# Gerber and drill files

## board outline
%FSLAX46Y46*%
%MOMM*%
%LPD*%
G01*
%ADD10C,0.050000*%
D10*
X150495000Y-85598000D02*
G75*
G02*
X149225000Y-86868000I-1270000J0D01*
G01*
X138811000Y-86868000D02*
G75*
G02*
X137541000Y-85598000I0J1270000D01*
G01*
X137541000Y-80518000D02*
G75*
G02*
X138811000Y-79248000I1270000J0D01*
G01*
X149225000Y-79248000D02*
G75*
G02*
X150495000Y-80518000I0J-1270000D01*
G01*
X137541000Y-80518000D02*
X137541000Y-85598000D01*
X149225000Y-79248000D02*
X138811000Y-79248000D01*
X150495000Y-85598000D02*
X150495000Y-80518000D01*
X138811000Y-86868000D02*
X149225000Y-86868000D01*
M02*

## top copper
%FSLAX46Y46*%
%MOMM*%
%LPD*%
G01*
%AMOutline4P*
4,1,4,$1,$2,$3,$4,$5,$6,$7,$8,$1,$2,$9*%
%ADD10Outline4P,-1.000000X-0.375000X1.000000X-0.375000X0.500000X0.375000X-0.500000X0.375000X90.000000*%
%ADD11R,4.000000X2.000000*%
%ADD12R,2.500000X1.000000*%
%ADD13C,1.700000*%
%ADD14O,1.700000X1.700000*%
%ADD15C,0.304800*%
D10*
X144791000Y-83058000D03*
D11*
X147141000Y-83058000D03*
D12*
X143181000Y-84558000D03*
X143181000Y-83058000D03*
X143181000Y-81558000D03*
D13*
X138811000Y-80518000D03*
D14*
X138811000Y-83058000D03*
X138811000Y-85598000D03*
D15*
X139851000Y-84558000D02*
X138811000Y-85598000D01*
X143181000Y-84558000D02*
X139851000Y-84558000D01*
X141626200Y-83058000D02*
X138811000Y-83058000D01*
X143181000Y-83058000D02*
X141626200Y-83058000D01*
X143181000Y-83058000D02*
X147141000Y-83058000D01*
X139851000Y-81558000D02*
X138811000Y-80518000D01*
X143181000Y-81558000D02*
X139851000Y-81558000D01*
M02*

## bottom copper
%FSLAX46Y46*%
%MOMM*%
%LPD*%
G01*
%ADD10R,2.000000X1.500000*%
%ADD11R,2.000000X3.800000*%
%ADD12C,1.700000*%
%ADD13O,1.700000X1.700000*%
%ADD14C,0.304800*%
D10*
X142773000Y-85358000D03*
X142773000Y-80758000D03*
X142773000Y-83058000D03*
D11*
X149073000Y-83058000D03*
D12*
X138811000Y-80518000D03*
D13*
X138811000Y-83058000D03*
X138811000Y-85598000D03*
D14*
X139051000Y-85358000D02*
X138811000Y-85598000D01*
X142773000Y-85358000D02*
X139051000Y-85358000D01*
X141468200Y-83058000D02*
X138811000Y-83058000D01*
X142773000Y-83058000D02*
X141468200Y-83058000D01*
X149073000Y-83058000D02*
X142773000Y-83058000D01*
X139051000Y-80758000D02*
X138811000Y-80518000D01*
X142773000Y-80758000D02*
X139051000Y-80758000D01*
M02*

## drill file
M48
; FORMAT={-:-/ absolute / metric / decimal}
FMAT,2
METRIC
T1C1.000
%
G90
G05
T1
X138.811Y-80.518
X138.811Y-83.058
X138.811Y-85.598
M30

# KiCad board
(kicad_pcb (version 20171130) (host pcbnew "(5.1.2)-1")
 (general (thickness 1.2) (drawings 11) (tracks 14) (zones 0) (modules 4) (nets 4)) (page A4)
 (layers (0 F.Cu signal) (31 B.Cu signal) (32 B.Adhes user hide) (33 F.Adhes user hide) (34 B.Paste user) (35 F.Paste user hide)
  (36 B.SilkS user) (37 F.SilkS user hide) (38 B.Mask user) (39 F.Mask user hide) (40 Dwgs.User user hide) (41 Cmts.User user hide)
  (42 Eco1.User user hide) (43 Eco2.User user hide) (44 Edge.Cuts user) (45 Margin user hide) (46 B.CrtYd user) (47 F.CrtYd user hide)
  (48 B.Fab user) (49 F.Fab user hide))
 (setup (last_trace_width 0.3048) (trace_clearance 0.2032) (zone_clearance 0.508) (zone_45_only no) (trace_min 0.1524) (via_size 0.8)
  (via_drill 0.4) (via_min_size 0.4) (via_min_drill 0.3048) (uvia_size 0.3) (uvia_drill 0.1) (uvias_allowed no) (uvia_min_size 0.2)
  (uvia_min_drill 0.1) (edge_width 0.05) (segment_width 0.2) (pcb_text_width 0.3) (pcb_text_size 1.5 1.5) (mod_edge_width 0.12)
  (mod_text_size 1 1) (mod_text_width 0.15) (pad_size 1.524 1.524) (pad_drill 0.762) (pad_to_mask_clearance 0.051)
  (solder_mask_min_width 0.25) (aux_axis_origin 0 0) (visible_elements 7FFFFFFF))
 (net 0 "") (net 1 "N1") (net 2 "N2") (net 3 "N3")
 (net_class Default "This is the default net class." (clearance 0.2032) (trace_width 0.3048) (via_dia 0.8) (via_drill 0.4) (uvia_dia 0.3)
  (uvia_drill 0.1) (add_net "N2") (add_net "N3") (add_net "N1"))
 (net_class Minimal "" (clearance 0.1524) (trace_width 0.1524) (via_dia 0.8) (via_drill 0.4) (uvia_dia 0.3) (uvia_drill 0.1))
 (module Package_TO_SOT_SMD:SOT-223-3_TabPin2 (layer B.Cu) (at 145.923 83.058)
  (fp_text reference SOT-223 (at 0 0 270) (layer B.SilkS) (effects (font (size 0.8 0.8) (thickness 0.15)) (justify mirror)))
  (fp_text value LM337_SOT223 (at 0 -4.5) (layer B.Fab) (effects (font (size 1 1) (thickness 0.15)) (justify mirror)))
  (pad 1 smd rect (at -3.15 2.3) (size 2 1.5) (layers B.Cu B.Paste B.Mask) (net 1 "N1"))
  (pad 3 smd rect (at -3.15 -2.3) (size 2 1.5) (layers B.Cu B.Paste B.Mask) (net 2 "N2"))
  (pad 2 smd rect (at -3.15 0) (size 2 1.5) (layers B.Cu B.Paste B.Mask) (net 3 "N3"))
  (pad 2 smd rect (at 3.15 0) (size 2 3.8) (layers B.Cu B.Paste B.Mask) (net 3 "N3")))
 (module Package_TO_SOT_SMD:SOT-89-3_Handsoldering (layer F.Cu) (at 145.161 83.058)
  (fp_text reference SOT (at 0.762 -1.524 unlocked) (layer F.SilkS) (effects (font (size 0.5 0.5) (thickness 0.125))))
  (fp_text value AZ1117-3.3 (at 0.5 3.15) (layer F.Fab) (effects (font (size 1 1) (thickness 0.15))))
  (pad 2 smd trapezoid (at -0.37 0 90) (size 1.5 0.75) (rect_delta 0 0.5) (layers F.Cu F.Paste F.Mask) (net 3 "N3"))
  (pad 2 smd rect (at 1.98 0 270) (size 2 4) (layers F.Cu F.Paste F.Mask) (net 3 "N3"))
  (pad 3 smd rect (at -1.98 1.5 270) (size 1 2.5) (layers F.Cu F.Paste F.Mask) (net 1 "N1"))
  (pad 2 smd rect (at -1.98 0 270) (size 1 2.5) (layers F.Cu F.Paste F.Mask) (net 3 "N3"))
  (pad 1 smd rect (at -1.98 -1.5 270) (size 1 2.5) (layers F.Cu F.Paste F.Mask) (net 2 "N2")))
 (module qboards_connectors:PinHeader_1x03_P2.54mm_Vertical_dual (layer F.Cu) (at 138.811 80.518)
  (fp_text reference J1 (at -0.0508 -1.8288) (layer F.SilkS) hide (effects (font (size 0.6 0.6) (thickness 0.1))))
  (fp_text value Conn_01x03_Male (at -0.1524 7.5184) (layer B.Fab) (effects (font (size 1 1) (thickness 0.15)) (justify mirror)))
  (pad 1 thru_hole circle (at 0 0) (size 1.7 1.7) (drill 1) (layers *.Cu *.Mask) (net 2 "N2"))
  (pad 2 thru_hole oval (at 0 2.54) (size 1.7 1.7) (drill 1) (layers *.Cu *.Mask) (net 3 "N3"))
  (pad 3 thru_hole oval (at 0 5.08) (size 1.7 1.7) (drill 1) (layers *.Cu *.Mask) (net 1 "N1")))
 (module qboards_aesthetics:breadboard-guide (layer F.Cu) (at 123.571 80.518)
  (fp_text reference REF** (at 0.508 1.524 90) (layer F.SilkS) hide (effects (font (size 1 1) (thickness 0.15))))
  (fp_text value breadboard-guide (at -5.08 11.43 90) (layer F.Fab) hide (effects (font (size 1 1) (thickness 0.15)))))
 (gr_arc (start 149.225 85.598) (end 149.225 86.868) (angle -90) (layer Edge.Cuts) (width 0.05))
 (gr_arc (start 138.811 85.598) (end 137.541 85.598) (angle -90) (layer Edge.Cuts) (width 0.05))
 (gr_arc (start 138.811 80.518) (end 138.811 79.248) (angle -90) (layer Edge.Cuts) (width 0.05))
 (gr_arc (start 149.225 80.518) (end 150.495 80.518) (angle -90) (layer Edge.Cuts) (width 0.05))
 (gr_line (start 137.541 80.518) (end 137.541 85.598) (layer Edge.Cuts) (width 0.05))
 (gr_line (start 149.225 79.248) (end 138.811 79.248) (layer Edge.Cuts) (width 0.05))
 (gr_line (start 150.495 85.598) (end 150.495 80.518) (layer Edge.Cuts) (width 0.05))
 (gr_line (start 138.811 86.868) (end 149.225 86.868) (layer Edge.Cuts) (width 0.05))
 (segment (start 139.051 85.358) (end 138.811 85.598) (width 0.3048) (layer B.Cu) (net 1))
 (segment (start 142.773 85.358) (end 139.051 85.358) (width 0.3048) (layer B.Cu) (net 1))
 (segment (start 139.851 84.558) (end 138.811 85.598) (width 0.3048) (layer F.Cu) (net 1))
 (segment (start 143.181 84.558) (end 139.851 84.558) (width 0.3048) (layer F.Cu) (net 1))
 (segment (start 141.4682 83.058) (end 138.811 83.058) (width 0.3048) (layer B.Cu) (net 3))
 (segment (start 142.773 83.058) (end 141.4682 83.058) (width 0.3048) (layer B.Cu) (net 3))
 (segment (start 141.6262 83.058) (end 138.811 83.058) (width 0.3048) (layer F.Cu) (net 3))
 (segment (start 143.181 83.058) (end 141.6262 83.058) (width 0.3048) (layer F.Cu) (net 3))
 (segment (start 143.181 83.058) (end 147.141 83.058) (width 0.3048) (layer F.Cu) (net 3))
 (segment (start 149.073 83.058) (end 142.773 83.058) (width 0.3048) (layer B.Cu) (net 3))
 (segment (start 139.051 80.758) (end 138.811 80.518) (width 0.3048) (layer B.Cu) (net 2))
 (segment (start 142.773 80.758) (end 139.051 80.758) (width 0.3048) (layer B.Cu) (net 2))
 (segment (start 139.851 81.558) (end 138.811 80.518) (width 0.3048) (layer F.Cu) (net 2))
 (segment (start 143.181 81.558) (end 139.851 81.558) (width 0.3048) (layer F.Cu) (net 2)))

